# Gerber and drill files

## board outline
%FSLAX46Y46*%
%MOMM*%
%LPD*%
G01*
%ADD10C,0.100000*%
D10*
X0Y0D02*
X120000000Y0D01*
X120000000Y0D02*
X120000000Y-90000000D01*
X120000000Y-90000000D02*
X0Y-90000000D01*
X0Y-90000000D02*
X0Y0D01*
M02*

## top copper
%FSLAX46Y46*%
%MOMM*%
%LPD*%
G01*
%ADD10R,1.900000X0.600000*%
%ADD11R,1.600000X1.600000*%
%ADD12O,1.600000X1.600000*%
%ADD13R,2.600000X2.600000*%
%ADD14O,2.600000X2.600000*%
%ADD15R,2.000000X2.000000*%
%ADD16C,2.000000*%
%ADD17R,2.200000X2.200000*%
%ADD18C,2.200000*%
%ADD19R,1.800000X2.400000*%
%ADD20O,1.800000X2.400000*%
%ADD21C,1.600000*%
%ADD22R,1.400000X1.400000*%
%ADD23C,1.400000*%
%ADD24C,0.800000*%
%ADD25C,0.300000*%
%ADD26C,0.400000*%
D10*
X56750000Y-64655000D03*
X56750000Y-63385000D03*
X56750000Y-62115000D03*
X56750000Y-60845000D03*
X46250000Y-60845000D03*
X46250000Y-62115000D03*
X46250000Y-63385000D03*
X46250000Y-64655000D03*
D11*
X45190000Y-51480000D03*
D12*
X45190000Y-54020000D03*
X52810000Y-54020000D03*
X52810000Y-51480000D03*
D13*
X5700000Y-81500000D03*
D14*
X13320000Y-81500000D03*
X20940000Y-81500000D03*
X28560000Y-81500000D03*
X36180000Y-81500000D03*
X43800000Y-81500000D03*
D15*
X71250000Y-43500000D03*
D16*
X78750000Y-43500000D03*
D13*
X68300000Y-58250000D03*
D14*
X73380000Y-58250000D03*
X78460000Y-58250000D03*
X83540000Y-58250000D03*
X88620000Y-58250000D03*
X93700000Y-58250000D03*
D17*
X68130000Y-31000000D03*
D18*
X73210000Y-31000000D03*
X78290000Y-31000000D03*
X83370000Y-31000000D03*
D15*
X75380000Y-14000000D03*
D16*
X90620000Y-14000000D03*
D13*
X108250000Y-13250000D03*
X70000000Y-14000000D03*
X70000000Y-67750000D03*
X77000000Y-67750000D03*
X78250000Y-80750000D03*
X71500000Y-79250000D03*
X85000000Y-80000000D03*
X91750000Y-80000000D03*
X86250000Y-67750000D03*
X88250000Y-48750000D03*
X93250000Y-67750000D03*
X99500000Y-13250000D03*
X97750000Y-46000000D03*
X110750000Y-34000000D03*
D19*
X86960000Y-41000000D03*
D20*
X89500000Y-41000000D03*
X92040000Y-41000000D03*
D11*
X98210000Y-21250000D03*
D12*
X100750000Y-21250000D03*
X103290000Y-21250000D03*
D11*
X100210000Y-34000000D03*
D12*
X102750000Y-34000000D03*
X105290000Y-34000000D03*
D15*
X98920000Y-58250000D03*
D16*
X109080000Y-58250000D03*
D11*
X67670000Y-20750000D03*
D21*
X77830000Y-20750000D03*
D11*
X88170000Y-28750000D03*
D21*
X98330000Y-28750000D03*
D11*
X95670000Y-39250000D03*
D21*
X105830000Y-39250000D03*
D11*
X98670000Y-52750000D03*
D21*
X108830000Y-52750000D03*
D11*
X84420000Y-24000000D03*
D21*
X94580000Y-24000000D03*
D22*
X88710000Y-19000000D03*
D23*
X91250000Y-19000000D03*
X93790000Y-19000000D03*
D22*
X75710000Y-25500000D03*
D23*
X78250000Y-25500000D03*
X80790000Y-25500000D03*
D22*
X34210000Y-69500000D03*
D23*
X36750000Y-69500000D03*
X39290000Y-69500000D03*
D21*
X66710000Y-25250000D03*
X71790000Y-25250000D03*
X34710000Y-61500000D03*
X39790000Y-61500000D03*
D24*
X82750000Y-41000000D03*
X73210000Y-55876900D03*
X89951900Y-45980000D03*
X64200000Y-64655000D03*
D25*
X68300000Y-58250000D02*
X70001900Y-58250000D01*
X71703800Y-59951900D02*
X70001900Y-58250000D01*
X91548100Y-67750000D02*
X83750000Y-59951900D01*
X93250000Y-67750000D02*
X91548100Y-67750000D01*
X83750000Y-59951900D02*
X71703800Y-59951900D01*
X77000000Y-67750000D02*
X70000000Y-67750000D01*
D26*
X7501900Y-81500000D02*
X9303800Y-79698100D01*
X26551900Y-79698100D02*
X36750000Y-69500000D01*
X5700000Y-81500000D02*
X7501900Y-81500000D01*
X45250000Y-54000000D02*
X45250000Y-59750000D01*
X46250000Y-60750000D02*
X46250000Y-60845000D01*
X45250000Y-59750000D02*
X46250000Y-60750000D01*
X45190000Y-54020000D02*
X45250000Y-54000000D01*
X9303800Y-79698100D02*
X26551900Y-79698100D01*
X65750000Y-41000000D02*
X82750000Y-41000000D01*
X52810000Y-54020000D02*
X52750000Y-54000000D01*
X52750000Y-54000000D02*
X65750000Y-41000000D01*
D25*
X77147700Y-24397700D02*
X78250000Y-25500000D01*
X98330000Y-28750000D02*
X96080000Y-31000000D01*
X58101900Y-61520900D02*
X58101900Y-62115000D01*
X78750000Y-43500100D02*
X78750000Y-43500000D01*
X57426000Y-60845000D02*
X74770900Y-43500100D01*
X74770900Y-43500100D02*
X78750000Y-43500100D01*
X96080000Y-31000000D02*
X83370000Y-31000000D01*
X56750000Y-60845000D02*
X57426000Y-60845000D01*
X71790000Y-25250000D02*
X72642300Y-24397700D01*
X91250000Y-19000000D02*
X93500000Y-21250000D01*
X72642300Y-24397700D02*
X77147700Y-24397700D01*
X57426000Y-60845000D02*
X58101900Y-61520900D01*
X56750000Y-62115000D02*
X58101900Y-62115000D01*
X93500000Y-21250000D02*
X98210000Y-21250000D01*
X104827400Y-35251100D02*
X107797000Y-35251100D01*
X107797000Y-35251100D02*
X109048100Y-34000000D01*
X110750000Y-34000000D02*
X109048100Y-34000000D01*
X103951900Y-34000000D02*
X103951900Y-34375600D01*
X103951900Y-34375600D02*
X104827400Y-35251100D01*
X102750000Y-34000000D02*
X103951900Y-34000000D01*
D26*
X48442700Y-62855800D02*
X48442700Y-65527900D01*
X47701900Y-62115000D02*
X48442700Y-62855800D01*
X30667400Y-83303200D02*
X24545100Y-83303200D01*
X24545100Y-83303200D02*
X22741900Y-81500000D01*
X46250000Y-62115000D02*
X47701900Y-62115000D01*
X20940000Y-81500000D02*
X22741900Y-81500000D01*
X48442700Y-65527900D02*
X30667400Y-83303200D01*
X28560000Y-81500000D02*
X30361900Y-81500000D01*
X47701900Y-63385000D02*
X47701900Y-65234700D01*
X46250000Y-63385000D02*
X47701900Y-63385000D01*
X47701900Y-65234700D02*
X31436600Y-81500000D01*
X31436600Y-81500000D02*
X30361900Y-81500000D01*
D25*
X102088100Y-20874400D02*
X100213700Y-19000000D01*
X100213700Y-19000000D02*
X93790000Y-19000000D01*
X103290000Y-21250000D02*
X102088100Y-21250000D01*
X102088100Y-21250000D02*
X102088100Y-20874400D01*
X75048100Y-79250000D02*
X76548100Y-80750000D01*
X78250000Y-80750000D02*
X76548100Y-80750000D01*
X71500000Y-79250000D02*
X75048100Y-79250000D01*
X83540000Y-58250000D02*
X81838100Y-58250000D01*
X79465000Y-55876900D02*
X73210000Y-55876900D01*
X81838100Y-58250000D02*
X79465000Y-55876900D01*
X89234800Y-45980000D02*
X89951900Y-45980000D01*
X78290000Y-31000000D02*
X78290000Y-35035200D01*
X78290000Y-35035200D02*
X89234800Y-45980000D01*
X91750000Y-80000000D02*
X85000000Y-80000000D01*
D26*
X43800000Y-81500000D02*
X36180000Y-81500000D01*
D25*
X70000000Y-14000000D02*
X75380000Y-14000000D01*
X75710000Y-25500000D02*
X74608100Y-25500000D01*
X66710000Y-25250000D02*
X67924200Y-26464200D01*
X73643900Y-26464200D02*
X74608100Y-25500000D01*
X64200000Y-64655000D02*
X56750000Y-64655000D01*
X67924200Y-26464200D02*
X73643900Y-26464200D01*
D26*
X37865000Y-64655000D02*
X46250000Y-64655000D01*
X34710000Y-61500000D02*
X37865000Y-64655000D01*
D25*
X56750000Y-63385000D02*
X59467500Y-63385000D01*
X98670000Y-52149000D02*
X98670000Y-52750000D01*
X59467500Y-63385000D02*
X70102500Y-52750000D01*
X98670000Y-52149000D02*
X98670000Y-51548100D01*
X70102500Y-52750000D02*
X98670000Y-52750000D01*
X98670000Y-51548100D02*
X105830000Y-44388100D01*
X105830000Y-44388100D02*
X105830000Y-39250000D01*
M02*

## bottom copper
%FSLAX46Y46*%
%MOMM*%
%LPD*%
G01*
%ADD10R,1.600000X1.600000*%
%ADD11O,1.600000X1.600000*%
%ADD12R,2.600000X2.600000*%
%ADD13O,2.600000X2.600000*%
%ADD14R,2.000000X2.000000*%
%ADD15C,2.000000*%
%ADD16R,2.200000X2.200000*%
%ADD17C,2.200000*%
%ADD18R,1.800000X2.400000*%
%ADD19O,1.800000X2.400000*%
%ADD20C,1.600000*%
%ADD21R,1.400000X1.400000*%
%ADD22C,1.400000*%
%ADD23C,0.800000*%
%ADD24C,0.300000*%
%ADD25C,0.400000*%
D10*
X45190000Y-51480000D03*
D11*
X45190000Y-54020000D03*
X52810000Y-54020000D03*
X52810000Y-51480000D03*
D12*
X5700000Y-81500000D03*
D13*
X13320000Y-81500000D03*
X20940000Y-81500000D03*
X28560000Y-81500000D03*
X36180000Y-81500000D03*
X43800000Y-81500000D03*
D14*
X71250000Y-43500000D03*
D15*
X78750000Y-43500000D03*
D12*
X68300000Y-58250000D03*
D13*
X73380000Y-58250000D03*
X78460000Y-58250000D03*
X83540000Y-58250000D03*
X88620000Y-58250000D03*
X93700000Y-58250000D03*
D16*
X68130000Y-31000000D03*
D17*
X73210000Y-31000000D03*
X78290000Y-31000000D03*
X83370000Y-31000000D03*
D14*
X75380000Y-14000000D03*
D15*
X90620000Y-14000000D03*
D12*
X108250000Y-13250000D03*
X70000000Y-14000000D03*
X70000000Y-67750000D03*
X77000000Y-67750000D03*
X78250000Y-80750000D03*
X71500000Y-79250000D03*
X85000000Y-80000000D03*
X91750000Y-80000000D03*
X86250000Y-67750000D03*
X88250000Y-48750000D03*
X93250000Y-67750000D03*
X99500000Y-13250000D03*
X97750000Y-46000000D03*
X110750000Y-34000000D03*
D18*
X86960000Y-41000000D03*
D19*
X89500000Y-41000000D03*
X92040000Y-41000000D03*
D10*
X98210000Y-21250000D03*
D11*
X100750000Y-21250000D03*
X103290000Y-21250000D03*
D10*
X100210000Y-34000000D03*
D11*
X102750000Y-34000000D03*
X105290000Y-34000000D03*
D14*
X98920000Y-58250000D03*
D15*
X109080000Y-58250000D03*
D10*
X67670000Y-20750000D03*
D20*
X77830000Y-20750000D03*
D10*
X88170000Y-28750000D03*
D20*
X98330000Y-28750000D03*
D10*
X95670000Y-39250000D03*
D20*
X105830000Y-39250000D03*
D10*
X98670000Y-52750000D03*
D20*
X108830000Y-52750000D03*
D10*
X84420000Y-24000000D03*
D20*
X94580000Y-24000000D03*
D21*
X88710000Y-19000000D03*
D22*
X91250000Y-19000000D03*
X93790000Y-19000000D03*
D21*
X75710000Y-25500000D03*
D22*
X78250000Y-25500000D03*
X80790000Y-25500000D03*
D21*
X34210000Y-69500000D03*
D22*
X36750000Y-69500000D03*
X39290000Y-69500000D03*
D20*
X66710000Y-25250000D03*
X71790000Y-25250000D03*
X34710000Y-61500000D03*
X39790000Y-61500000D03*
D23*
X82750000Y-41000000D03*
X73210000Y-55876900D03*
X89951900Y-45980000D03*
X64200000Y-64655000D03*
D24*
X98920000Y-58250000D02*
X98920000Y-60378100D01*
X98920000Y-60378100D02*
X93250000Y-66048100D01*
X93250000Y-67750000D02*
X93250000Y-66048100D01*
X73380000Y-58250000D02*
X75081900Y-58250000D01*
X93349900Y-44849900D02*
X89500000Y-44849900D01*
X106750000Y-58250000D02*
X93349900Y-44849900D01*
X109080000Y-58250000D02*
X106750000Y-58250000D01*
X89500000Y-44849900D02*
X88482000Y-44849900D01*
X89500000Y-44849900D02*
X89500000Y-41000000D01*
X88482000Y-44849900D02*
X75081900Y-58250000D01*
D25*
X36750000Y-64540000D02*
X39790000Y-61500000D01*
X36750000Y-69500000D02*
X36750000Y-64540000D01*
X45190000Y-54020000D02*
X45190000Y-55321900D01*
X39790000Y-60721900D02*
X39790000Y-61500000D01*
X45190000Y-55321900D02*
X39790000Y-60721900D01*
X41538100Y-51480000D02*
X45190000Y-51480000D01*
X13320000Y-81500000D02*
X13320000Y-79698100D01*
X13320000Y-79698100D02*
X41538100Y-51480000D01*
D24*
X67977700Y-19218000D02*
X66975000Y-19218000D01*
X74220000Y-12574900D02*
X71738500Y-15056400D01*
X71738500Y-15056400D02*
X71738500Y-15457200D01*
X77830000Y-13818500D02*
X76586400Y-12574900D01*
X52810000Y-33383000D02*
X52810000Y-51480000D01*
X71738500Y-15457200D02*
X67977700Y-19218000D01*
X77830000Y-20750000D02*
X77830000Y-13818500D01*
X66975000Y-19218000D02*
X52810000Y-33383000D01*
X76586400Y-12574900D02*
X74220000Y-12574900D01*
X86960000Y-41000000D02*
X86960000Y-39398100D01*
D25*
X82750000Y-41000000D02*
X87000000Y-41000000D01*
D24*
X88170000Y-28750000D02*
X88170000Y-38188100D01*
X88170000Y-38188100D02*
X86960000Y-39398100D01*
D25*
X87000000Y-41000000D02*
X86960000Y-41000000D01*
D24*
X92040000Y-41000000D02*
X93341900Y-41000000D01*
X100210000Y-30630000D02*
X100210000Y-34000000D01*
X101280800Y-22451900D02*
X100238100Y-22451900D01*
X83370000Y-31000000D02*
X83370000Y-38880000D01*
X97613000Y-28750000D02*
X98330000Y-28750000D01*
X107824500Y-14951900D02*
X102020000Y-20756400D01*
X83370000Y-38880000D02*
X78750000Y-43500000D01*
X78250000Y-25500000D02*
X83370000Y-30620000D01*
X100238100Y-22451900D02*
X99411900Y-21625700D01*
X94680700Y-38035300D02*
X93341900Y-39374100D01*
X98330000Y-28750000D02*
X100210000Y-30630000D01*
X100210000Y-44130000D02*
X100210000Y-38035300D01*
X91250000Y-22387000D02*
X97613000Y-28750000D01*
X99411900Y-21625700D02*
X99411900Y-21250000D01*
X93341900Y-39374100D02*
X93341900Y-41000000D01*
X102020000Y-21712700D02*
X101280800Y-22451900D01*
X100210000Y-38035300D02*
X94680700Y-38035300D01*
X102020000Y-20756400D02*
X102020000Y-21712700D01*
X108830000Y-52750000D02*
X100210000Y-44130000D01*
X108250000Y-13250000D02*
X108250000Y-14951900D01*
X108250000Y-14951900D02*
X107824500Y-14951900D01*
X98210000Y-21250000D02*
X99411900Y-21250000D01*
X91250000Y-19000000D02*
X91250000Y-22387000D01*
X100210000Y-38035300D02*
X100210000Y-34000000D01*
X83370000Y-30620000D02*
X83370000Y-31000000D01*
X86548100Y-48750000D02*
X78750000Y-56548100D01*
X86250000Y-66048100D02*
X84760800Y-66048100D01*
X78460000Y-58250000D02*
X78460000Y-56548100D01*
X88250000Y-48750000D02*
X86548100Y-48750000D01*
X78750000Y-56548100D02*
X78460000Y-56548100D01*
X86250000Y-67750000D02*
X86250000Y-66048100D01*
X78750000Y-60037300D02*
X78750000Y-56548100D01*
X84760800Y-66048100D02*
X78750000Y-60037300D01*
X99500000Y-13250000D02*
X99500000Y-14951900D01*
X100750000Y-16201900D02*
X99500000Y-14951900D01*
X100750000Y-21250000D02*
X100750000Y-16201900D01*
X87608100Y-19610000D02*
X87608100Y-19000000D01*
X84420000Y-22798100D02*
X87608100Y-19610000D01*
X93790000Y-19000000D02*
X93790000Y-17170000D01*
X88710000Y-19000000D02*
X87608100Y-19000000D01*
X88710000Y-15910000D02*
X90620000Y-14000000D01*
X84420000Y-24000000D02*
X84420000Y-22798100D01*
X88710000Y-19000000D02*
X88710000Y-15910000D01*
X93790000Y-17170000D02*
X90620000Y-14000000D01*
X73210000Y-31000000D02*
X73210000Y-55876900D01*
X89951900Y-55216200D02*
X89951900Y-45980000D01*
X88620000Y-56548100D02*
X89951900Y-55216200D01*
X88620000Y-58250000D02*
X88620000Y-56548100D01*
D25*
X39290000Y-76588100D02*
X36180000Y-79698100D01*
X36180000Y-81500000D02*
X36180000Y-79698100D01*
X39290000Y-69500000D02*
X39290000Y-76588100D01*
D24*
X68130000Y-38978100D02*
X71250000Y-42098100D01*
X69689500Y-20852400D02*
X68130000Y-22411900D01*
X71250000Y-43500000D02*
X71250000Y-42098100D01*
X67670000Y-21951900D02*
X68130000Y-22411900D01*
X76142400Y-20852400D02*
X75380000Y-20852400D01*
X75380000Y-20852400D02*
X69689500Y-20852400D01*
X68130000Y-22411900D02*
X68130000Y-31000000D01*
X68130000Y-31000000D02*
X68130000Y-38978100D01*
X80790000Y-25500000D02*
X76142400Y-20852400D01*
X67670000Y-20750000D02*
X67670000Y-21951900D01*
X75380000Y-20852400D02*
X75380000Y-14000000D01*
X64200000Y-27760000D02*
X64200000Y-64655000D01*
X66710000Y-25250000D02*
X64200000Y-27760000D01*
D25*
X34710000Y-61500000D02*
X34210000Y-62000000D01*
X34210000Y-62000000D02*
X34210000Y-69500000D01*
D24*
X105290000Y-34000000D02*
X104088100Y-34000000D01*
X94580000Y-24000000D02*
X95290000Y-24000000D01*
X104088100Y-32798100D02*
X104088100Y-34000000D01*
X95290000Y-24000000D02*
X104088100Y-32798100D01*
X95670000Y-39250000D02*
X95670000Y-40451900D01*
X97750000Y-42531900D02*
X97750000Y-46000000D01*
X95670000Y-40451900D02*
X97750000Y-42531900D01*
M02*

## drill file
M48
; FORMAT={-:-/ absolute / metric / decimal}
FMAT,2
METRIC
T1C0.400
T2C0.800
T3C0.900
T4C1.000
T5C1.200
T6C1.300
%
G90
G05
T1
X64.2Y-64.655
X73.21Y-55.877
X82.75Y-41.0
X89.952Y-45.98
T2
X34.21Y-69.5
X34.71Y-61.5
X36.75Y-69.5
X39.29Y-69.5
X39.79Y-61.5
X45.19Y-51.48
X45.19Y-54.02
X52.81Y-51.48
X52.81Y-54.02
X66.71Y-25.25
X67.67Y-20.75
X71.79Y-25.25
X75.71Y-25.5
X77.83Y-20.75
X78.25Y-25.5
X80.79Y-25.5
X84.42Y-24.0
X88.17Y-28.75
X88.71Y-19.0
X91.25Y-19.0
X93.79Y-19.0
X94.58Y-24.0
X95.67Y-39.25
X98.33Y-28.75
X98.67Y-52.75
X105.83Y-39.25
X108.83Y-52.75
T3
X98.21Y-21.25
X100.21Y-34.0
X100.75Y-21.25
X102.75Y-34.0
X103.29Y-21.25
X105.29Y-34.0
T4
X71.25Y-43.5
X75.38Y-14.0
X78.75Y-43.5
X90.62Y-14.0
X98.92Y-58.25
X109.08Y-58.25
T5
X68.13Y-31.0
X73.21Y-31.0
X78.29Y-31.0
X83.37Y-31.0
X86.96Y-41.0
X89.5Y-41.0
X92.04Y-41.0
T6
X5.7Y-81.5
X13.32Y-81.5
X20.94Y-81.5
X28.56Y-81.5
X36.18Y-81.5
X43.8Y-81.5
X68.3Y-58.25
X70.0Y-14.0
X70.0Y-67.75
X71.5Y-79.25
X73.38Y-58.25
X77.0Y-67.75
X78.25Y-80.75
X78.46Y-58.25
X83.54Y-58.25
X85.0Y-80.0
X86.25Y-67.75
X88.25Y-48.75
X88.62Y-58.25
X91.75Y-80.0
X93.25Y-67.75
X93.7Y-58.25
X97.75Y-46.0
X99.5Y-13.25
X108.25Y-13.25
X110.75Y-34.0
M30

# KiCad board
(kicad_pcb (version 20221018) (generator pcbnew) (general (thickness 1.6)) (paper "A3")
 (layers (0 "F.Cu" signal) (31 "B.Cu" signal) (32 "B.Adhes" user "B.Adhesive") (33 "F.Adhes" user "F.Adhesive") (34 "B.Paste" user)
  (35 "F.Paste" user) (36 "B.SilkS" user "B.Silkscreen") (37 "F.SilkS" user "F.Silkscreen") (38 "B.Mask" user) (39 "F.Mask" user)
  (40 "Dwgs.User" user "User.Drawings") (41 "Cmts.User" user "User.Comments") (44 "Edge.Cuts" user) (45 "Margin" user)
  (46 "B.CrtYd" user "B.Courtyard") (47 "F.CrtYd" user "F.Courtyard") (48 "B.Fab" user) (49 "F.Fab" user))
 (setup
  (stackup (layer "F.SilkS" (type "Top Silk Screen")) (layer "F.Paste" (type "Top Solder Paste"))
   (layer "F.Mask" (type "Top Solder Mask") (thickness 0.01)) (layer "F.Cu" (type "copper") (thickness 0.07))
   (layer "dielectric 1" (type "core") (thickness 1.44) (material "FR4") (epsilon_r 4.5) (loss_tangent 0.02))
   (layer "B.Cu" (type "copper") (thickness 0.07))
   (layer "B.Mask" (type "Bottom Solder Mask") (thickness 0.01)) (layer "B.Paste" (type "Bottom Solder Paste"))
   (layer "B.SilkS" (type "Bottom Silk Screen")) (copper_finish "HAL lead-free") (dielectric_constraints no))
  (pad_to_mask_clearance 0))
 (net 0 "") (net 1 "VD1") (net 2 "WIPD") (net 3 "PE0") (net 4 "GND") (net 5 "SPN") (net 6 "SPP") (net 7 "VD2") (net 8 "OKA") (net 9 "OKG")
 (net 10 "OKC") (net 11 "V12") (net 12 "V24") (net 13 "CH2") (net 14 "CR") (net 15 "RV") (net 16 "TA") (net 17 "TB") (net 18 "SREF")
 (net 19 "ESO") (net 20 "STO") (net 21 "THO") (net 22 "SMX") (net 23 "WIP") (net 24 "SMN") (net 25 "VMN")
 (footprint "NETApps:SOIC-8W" (layer "F.Cu") (at 51.5 62.75 180)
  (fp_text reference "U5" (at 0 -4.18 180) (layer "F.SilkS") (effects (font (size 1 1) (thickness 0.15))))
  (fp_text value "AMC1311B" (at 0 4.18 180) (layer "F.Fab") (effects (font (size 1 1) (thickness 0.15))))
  (pad "1" smd rect (at -5.25 -1.905) (size 1.9 0.6) (layers "F.Cu" "F.Paste" "F.Mask") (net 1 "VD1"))
  (pad "2" smd rect (at -5.25 -0.635) (size 1.9 0.6) (layers "F.Cu" "F.Paste" "F.Mask") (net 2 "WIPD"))
  (pad "3" smd rect (at -5.25 0.635) (size 1.9 0.6) (layers "F.Cu" "F.Paste" "F.Mask") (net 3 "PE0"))
  (pad "4" smd rect (at -5.25 1.905) (size 1.9 0.6) (layers "F.Cu" "F.Paste" "F.Mask") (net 3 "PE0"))
  (pad "5" smd rect (at 5.25 1.905) (size 1.9 0.6) (layers "F.Cu" "F.Paste" "F.Mask") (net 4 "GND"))
  (pad "6" smd rect (at 5.25 0.635) (size 1.9 0.6) (layers "F.Cu" "F.Paste" "F.Mask") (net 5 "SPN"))
  (pad "7" smd rect (at 5.25 -0.635) (size 1.9 0.6) (layers "F.Cu" "F.Paste" "F.Mask") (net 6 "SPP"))
  (pad "8" smd rect (at 5.25 -1.905) (size 1.9 0.6) (layers "F.Cu" "F.Paste" "F.Mask") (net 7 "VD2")))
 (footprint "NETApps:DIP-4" (layer "F.Cu") (at 49 52.75)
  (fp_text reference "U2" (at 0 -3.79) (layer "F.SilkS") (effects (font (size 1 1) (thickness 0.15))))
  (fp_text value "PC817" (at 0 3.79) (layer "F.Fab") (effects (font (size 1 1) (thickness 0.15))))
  (pad "1" thru_hole rect (at -3.81 -1.27) (size 1.6 1.6) (drill 0.8) (layers "*.Cu" "*.Mask") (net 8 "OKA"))
  (pad "2" thru_hole oval (at -3.81 1.27) (size 1.6 1.6) (drill 0.8) (layers "*.Cu" "*.Mask") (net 4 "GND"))
  (pad "3" thru_hole oval (at 3.81 1.27) (size 1.6 1.6) (drill 0.8) (layers "*.Cu" "*.Mask") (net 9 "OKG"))
  (pad "4" thru_hole oval (at 3.81 -1.27) (size 1.6 1.6) (drill 0.8) (layers "*.Cu" "*.Mask") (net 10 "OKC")))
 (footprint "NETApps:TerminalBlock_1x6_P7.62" (layer "F.Cu") (at 24.75 81.5)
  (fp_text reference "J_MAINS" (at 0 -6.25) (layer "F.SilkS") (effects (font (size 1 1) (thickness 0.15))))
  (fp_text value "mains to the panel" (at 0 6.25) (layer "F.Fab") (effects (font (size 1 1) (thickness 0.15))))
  (pad "1" thru_hole rect (at -19.05 0) (size 2.6 2.6) (drill 1.3) (layers "*.Cu" "*.Mask") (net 4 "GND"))
  (pad "2" thru_hole oval (at -11.43 0) (size 2.6 2.6) (drill 1.3) (layers "*.Cu" "*.Mask") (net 8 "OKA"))
  (pad "3" thru_hole oval (at -3.81 0) (size 2.6 2.6) (drill 1.3) (layers "*.Cu" "*.Mask") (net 5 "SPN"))
  (pad "4" thru_hole oval (at 3.81 0) (size 2.6 2.6) (drill 1.3) (layers "*.Cu" "*.Mask") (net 6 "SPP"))
  (pad "5" thru_hole oval (at 11.43 0) (size 2.6 2.6) (drill 1.3) (layers "*.Cu" "*.Mask") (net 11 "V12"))
  (pad "6" thru_hole oval (at 19.05 0) (size 2.6 2.6) (drill 1.3) (layers "*.Cu" "*.Mask") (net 11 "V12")))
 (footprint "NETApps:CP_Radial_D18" (layer "F.Cu") (at 75 43.5)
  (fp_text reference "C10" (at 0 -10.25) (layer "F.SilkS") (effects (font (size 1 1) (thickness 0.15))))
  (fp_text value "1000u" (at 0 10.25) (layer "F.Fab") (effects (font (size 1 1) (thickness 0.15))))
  (pad "1" thru_hole rect (at -3.75 0) (size 2 2) (drill 1) (layers "*.Cu" "*.Mask") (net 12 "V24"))
  (pad "2" thru_hole circle (at 3.75 0) (size 2 2) (drill 1) (layers "*.Cu" "*.Mask") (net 3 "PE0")))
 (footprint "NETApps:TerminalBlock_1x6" (layer "F.Cu") (at 81 58.25)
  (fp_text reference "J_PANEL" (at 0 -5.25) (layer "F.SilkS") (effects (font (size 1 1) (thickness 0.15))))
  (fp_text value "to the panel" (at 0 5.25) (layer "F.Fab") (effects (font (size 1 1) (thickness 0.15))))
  (pad "1" thru_hole rect (at -12.7 0) (size 2.6 2.6) (drill 1.3) (layers "*.Cu" "*.Mask") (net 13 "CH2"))
  (pad "2" thru_hole oval (at -7.62 0) (size 2.6 2.6) (drill 1.3) (layers "*.Cu" "*.Mask") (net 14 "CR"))
  (pad "3" thru_hole oval (at -2.54 0) (size 2.6 2.6) (drill 1.3) (layers "*.Cu" "*.Mask") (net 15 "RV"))
  (pad "4" thru_hole oval (at 2.54 0) (size 2.6 2.6) (drill 1.3) (layers "*.Cu" "*.Mask") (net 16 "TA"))
  (pad "5" thru_hole oval (at 7.62 0) (size 2.6 2.6) (drill 1.3) (layers "*.Cu" "*.Mask") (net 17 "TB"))
  (pad "6" thru_hole oval (at 12.7 0) (size 2.6 2.6) (drill 1.3) (layers "*.Cu" "*.Mask")))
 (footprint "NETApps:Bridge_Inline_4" (layer "F.Cu") (at 75.75 31)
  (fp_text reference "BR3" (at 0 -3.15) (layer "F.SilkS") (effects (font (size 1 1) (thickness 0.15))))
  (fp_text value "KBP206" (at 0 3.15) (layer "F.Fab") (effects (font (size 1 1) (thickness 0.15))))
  (pad "1" thru_hole rect (at -7.62 0) (size 2.2 2.2) (drill 1.2) (layers "*.Cu" "*.Mask") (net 12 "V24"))
  (pad "2" thru_hole circle (at -2.54 0) (size 2.2 2.2) (drill 1.2) (layers "*.Cu" "*.Mask") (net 16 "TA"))
  (pad "3" thru_hole circle (at 2.54 0) (size 2.2 2.2) (drill 1.2) (layers "*.Cu" "*.Mask") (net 17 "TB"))
  (pad "4" thru_hole circle (at 7.62 0) (size 2.2 2.2) (drill 1.2) (layers "*.Cu" "*.Mask") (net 3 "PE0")))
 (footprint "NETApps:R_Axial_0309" (layer "F.Cu") (at 83 14)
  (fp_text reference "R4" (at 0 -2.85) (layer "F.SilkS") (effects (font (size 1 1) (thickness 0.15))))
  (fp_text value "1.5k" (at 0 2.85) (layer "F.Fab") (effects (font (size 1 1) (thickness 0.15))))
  (pad "1" thru_hole rect (at -7.62 0) (size 2 2) (drill 1) (layers "*.Cu" "*.Mask") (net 12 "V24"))
  (pad "2" thru_hole circle (at 7.62 0) (size 2 2) (drill 1) (layers "*.Cu" "*.Mask") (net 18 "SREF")))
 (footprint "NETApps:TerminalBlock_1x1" (layer "F.Cu") (at 108.25 13.25)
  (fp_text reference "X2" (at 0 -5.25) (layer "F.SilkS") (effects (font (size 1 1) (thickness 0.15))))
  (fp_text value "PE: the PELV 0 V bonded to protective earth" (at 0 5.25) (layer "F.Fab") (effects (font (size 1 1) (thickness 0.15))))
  (pad "1" thru_hole rect (at 0 0) (size 2.6 2.6) (drill 1.3) (layers "*.Cu" "*.Mask") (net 3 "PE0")))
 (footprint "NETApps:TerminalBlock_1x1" (layer "F.Cu") (at 70 14)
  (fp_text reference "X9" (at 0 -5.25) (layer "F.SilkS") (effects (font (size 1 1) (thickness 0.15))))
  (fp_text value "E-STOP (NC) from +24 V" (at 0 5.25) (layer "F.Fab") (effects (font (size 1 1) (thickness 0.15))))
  (pad "1" thru_hole rect (at 0 0) (size 2.6 2.6) (drill 1.3) (layers "*.Cu" "*.Mask") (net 12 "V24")))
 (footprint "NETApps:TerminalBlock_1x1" (layer "F.Cu") (at 70 67.75)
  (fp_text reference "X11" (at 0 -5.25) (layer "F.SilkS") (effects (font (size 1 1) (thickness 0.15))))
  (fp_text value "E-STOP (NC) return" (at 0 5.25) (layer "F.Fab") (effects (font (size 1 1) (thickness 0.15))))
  (pad "1" thru_hole rect (at 0 0) (size 2.6 2.6) (drill 1.3) (layers "*.Cu" "*.Mask") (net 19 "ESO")))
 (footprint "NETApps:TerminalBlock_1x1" (layer "F.Cu") (at 77 67.75)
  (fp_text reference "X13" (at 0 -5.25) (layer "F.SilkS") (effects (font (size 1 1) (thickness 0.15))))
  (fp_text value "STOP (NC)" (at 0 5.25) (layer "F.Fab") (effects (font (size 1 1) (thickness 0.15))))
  (pad "1" thru_hole rect (at 0 0) (size 2.6 2.6) (drill 1.3) (layers "*.Cu" "*.Mask") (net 19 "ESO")))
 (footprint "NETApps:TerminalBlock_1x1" (layer "F.Cu") (at 78.25 80.75)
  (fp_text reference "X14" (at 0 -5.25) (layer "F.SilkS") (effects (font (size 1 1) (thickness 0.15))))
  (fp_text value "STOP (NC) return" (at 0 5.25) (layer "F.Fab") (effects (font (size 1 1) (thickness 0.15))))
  (pad "1" thru_hole rect (at 0 0) (size 2.6 2.6) (drill 1.3) (layers "*.Cu" "*.Mask") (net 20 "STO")))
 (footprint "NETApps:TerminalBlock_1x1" (layer "F.Cu") (at 71.5 79.25)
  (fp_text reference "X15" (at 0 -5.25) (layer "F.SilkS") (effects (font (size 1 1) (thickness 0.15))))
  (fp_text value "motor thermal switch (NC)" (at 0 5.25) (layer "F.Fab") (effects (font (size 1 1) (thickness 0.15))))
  (pad "1" thru_hole rect (at 0 0) (size 2.6 2.6) (drill 1.3) (layers "*.Cu" "*.Mask") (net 20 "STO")))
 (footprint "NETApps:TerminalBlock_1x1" (layer "F.Cu") (at 85 80)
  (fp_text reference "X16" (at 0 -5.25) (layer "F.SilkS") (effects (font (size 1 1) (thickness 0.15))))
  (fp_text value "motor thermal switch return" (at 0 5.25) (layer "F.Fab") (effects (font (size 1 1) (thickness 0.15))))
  (pad "1" thru_hole rect (at 0 0) (size 2.6 2.6) (drill 1.3) (layers "*.Cu" "*.Mask") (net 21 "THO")))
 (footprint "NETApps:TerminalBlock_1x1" (layer "F.Cu") (at 91.75 80)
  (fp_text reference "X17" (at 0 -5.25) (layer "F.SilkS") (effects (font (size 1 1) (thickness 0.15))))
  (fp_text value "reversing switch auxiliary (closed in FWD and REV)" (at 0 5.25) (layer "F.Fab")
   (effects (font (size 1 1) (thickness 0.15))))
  (pad "1" thru_hole rect (at 0 0) (size 2.6 2.6) (drill 1.3) (layers "*.Cu" "*.Mask") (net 21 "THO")))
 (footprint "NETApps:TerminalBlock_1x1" (layer "F.Cu") (at 86.25 67.75)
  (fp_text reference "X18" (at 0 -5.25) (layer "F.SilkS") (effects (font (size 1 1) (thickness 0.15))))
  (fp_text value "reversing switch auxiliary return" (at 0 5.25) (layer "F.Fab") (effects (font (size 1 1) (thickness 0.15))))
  (pad "1" thru_hole rect (at 0 0) (size 2.6 2.6) (drill 1.3) (layers "*.Cu" "*.Mask") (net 15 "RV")))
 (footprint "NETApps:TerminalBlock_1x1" (layer "F.Cu") (at 88.25 48.75)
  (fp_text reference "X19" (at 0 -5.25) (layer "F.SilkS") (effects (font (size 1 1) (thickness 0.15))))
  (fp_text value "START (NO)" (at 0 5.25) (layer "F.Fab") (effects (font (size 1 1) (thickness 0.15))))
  (pad "1" thru_hole rect (at 0 0) (size 2.6 2.6) (drill 1.3) (layers "*.Cu" "*.Mask") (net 15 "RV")))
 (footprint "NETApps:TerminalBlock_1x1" (layer "F.Cu") (at 93.25 67.75)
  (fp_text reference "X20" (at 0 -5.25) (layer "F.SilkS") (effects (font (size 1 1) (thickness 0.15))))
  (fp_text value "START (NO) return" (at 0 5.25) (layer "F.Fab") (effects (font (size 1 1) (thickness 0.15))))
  (pad "1" thru_hole rect (at 0 0) (size 2.6 2.6) (drill 1.3) (layers "*.Cu" "*.Mask") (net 13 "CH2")))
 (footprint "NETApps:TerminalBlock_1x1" (layer "F.Cu") (at 99.5 13.25)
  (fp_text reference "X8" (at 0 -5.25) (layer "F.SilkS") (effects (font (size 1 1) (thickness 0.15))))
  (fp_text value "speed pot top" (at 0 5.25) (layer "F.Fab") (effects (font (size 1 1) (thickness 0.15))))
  (pad "1" thru_hole rect (at 0 0) (size 2.6 2.6) (drill 1.3) (layers "*.Cu" "*.Mask") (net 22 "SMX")))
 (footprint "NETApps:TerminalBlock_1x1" (layer "F.Cu") (at 97.75 46)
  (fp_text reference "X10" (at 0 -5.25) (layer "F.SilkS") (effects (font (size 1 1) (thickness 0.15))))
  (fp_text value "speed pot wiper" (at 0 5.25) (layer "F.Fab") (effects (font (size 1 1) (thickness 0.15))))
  (pad "1" thru_hole rect (at 0 0) (size 2.6 2.6) (drill 1.3) (layers "*.Cu" "*.Mask") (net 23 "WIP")))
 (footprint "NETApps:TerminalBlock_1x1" (layer "F.Cu") (at 110.75 34)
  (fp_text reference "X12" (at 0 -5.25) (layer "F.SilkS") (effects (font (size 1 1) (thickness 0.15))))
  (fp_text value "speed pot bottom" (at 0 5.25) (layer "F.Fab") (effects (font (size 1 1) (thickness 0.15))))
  (pad "1" thru_hole rect (at 0 0) (size 2.6 2.6) (drill 1.3) (layers "*.Cu" "*.Mask") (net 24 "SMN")))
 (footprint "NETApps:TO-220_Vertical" (layer "F.Cu") (at 89.5 41)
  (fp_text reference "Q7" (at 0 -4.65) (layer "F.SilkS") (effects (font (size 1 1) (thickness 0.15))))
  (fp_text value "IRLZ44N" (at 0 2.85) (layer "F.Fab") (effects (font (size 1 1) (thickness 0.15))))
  (pad "1" thru_hole rect (at -2.54 0) (size 1.8 2.4) (drill 1.2) (layers "*.Cu" "*.Mask") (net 9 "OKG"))
  (pad "2" thru_hole oval (at 0 0) (size 1.8 2.4) (drill 1.2) (layers "*.Cu" "*.Mask") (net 14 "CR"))
  (pad "3" thru_hole oval (at 2.54 0) (size 1.8 2.4) (drill 1.2) (layers "*.Cu" "*.Mask") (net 3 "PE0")))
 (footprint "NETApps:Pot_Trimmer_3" (layer "F.Cu") (at 100.75 21.25)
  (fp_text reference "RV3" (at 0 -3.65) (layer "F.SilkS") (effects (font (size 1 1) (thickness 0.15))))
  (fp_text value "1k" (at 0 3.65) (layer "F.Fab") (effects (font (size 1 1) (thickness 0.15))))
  (pad "1" thru_hole rect (at -2.54 0) (size 1.6 1.6) (drill 0.9) (layers "*.Cu" "*.Mask") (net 3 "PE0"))
  (pad "2" thru_hole oval (at 0 0) (size 1.6 1.6) (drill 0.9) (layers "*.Cu" "*.Mask") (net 22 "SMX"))
  (pad "3" thru_hole oval (at 2.54 0) (size 1.6 1.6) (drill 0.9) (layers "*.Cu" "*.Mask") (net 18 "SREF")))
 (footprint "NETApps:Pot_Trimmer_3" (layer "F.Cu") (at 102.75 34)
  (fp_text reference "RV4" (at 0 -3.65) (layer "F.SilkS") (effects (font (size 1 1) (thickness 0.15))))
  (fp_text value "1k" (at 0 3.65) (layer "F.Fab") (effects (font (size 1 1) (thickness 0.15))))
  (pad "1" thru_hole rect (at -2.54 0) (size 1.6 1.6) (drill 0.9) (layers "*.Cu" "*.Mask") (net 3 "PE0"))
  (pad "2" thru_hole oval (at 0 0) (size 1.6 1.6) (drill 0.9) (layers "*.Cu" "*.Mask") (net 24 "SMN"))
  (pad "3" thru_hole oval (at 2.54 0) (size 1.6 1.6) (drill 0.9) (layers "*.Cu" "*.Mask") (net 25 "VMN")))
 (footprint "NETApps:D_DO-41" (layer "F.Cu") (at 104 58.25)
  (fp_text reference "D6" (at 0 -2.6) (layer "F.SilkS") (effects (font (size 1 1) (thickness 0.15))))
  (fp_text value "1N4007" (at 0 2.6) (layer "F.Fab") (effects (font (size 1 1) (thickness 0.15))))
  (pad "1" thru_hole rect (at -5.08 0) (size 2 2) (drill 1) (layers "*.Cu" "*.Mask") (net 13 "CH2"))
  (pad "2" thru_hole circle (at 5.08 0) (size 2 2) (drill 1) (layers "*.Cu" "*.Mask") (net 14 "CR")))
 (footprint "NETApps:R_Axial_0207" (layer "F.Cu") (at 72.75 20.75)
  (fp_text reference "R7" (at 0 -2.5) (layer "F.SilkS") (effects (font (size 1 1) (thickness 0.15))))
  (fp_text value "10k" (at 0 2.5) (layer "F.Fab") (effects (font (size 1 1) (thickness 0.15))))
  (pad "1" thru_hole rect (at -5.08 0) (size 1.6 1.6) (drill 0.8) (layers "*.Cu" "*.Mask") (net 12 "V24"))
  (pad "2" thru_hole circle (at 5.08 0) (size 1.6 1.6) (drill 0.8) (layers "*.Cu" "*.Mask") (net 10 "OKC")))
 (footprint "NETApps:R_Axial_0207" (layer "F.Cu") (at 93.25 28.75)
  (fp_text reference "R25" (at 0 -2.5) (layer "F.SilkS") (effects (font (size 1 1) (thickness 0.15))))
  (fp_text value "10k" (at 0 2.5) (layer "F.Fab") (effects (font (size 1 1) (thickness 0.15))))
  (pad "1" thru_hole rect (at -5.08 0) (size 1.6 1.6) (drill 0.8) (layers "*.Cu" "*.Mask") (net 9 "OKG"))
  (pad "2" thru_hole circle (at 5.08 0) (size 1.6 1.6) (drill 0.8) (layers "*.Cu" "*.Mask") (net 3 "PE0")))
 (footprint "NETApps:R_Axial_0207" (layer "F.Cu") (at 100.75 39.25)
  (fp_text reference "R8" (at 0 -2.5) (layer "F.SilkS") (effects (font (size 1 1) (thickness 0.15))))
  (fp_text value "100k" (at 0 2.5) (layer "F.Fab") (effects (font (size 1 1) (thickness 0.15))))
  (pad "1" thru_hole rect (at -5.08 0) (size 1.6 1.6) (drill 0.8) (layers "*.Cu" "*.Mask") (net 23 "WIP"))
  (pad "2" thru_hole circle (at 5.08 0) (size 1.6 1.6) (drill 0.8) (layers "*.Cu" "*.Mask") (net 2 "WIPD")))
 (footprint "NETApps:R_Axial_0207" (layer "F.Cu") (at 103.75 52.75)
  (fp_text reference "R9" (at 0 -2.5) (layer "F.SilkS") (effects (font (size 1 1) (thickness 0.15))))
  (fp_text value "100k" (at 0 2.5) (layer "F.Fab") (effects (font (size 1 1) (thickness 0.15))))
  (pad "1" thru_hole rect (at -5.08 0) (size 1.6 1.6) (drill 0.8) (layers "*.Cu" "*.Mask") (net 2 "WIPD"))
  (pad "2" thru_hole circle (at 5.08 0) (size 1.6 1.6) (drill 0.8) (layers "*.Cu" "*.Mask") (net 3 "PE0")))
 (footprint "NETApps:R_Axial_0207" (layer "F.Cu") (at 89.5 24)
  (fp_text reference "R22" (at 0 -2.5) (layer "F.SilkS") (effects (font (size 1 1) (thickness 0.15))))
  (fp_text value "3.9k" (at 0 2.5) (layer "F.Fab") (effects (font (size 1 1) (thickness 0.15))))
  (pad "1" thru_hole rect (at -5.08 0) (size 1.6 1.6) (drill 0.8) (layers "*.Cu" "*.Mask") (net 18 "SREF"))
  (pad "2" thru_hole circle (at 5.08 0) (size 1.6 1.6) (drill 0.8) (layers "*.Cu" "*.Mask") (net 25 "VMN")))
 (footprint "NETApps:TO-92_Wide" (layer "F.Cu") (at 91.25 19)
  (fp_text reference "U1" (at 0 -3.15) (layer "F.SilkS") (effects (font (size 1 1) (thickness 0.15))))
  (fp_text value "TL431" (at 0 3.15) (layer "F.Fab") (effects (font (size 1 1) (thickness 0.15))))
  (pad "1" thru_hole rect (at -2.54 0) (size 1.4 1.4) (drill 0.8) (layers "*.Cu" "*.Mask") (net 18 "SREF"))
  (pad "2" thru_hole circle (at 0 0) (size 1.4 1.4) (drill 0.8) (layers "*.Cu" "*.Mask") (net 3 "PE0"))
  (pad "3" thru_hole circle (at 2.54 0) (size 1.4 1.4) (drill 0.8) (layers "*.Cu" "*.Mask") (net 18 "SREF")))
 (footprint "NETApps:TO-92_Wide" (layer "F.Cu") (at 78.25 25.5)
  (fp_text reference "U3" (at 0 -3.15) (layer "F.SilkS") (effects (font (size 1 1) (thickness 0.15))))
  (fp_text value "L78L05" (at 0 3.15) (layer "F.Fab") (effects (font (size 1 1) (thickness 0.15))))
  (pad "1" thru_hole rect (at -2.54 0) (size 1.4 1.4) (drill 0.8) (layers "*.Cu" "*.Mask") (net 1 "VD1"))
  (pad "2" thru_hole circle (at 0 0) (size 1.4 1.4) (drill 0.8) (layers "*.Cu" "*.Mask") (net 3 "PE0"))
  (pad "3" thru_hole circle (at 2.54 0) (size 1.4 1.4) (drill 0.8) (layers "*.Cu" "*.Mask") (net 12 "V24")))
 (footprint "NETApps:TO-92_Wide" (layer "F.Cu") (at 36.75 69.5)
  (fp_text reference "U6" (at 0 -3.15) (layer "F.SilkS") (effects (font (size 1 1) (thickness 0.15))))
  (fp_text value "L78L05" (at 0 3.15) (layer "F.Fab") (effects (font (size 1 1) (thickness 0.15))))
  (pad "1" thru_hole rect (at -2.54 0) (size 1.4 1.4) (drill 0.8) (layers "*.Cu" "*.Mask") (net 7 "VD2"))
  (pad "2" thru_hole circle (at 0 0) (size 1.4 1.4) (drill 0.8) (layers "*.Cu" "*.Mask") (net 4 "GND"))
  (pad "3" thru_hole circle (at 2.54 0) (size 1.4 1.4) (drill 0.8) (layers "*.Cu" "*.Mask") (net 11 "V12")))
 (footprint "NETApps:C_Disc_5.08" (layer "F.Cu") (at 69.25 25.25)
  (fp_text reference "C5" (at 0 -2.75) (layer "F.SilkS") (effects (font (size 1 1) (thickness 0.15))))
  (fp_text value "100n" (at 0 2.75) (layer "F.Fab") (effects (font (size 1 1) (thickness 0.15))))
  (pad "1" thru_hole circle (at -2.54 0) (size 1.6 1.6) (drill 0.8) (layers "*.Cu" "*.Mask") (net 1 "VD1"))
  (pad "2" thru_hole circle (at 2.54 0) (size 1.6 1.6) (drill 0.8) (layers "*.Cu" "*.Mask") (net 3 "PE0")))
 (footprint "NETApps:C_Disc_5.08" (layer "F.Cu") (at 37.25 61.5)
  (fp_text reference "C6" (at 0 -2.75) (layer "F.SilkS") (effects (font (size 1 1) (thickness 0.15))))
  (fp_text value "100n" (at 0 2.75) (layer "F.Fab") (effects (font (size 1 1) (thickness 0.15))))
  (pad "1" thru_hole circle (at -2.54 0) (size 1.6 1.6) (drill 0.8) (layers "*.Cu" "*.Mask") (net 7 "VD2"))
  (pad "2" thru_hole circle (at 2.54 0) (size 1.6 1.6) (drill 0.8) (layers "*.Cu" "*.Mask") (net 4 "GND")))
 (gr_line (start 0 0) (end 120 0) (stroke (width 0.1) (type solid)) (layer "Edge.Cuts"))
 (gr_line (start 120 0) (end 120 90) (stroke (width 0.1) (type solid)) (layer "Edge.Cuts"))
 (gr_line (start 120 90) (end 0 90) (stroke (width 0.1) (type solid)) (layer "Edge.Cuts"))
 (gr_line (start 0 90) (end 0 0) (stroke (width 0.1) (type solid)) (layer "Edge.Cuts"))
 (segment (start 68.3 58.25) (end 70.0019 58.25) (width 0.3) (layer "F.Cu") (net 13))
 (segment (start 71.7038 59.9519) (end 70.0019 58.25) (width 0.3) (layer "F.Cu") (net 13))
 (segment (start 91.5481 67.75) (end 83.75 59.9519) (width 0.3) (layer "F.Cu") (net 13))
 (segment (start 93.25 67.75) (end 91.5481 67.75) (width 0.3) (layer "F.Cu") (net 13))
 (segment (start 83.75 59.9519) (end 71.7038 59.9519) (width 0.3) (layer "F.Cu") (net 13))
 (segment (start 98.92 58.25) (end 98.92 60.3781) (width 0.3) (layer "B.Cu") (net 13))
 (segment (start 98.92 60.3781) (end 93.25 66.0481) (width 0.3) (layer "B.Cu") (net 13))
 (segment (start 93.25 67.75) (end 93.25 66.0481) (width 0.3) (layer "B.Cu") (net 13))
 (segment (start 73.38 58.25) (end 75.0819 58.25) (width 0.3) (layer "B.Cu") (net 14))
 (segment (start 93.3499 44.8499) (end 89.5 44.8499) (width 0.3) (layer "B.Cu") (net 14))
 (segment (start 106.75 58.25) (end 93.3499 44.8499) (width 0.3) (layer "B.Cu") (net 14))
 (segment (start 109.08 58.25) (end 106.75 58.25) (width 0.3) (layer "B.Cu") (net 14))
 (segment (start 89.5 44.8499) (end 88.482 44.8499) (width 0.3) (layer "B.Cu") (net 14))
 (segment (start 89.5 44.8499) (end 89.5 41) (width 0.3) (layer "B.Cu") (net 14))
 (segment (start 88.482 44.8499) (end 75.0819 58.25) (width 0.3) (layer "B.Cu") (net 14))
 (segment (start 77 67.75) (end 70 67.75) (width 0.3) (layer "F.Cu") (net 19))
 (segment locked (start 7.5019 81.5) (end 9.3038 79.6981) (width 0.4) (layer "F.Cu") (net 4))
 (segment locked (start 26.5519 79.6981) (end 36.75 69.5) (width 0.4) (layer "F.Cu") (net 4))
 (segment locked (start 5.7 81.5) (end 7.5019 81.5) (width 0.4) (layer "F.Cu") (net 4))
 (segment locked (start 45.25 54) (end 45.25 59.75) (width 0.4) (layer "F.Cu") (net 4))
 (segment locked (start 46.25 60.75) (end 46.25 60.845) (width 0.4) (layer "F.Cu") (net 4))
 (segment locked (start 45.25 59.75) (end 46.25 60.75) (width 0.4) (layer "F.Cu") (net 4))
 (segment locked (start 45.19 54.02) (end 45.25 54) (width 0.4) (layer "F.Cu") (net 4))
 (segment locked (start 9.3038 79.6981) (end 26.5519 79.6981) (width 0.4) (layer "F.Cu") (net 4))
 (segment locked (start 36.75 64.54) (end 39.79 61.5) (width 0.4) (layer "B.Cu") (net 4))
 (segment locked (start 36.75 69.5) (end 36.75 64.54) (width 0.4) (layer "B.Cu") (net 4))
 (segment locked (start 45.19 54.02) (end 45.19 55.3219) (width 0.4) (layer "B.Cu") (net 4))
 (segment locked (start 39.79 60.7219) (end 39.79 61.5) (width 0.4) (layer "B.Cu") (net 4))
 (segment locked (start 45.19 55.3219) (end 39.79 60.7219) (width 0.4) (layer "B.Cu") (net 4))
 (segment locked (start 41.5381 51.48) (end 45.19 51.48) (width 0.4) (layer "B.Cu") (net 8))
 (segment locked (start 13.32 81.5) (end 13.32 79.6981) (width 0.4) (layer "B.Cu") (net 8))
 (segment locked (start 13.32 79.6981) (end 41.5381 51.48) (width 0.4) (layer "B.Cu") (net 8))
 (segment (start 67.9777 19.218) (end 66.975 19.218) (width 0.3) (layer "B.Cu") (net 10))
 (segment (start 74.22 12.5749) (end 71.7385 15.0564) (width 0.3) (layer "B.Cu") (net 10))
 (segment (start 71.7385 15.0564) (end 71.7385 15.4572) (width 0.3) (layer "B.Cu") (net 10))
 (segment (start 77.83 13.8185) (end 76.5864 12.5749) (width 0.3) (layer "B.Cu") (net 10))
 (segment (start 52.81 33.383) (end 52.81 51.48) (width 0.3) (layer "B.Cu") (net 10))
 (segment (start 71.7385 15.4572) (end 67.9777 19.218) (width 0.3) (layer "B.Cu") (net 10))
 (segment (start 77.83 20.75) (end 77.83 13.8185) (width 0.3) (layer "B.Cu") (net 10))
 (segment (start 66.975 19.218) (end 52.81 33.383) (width 0.3) (layer "B.Cu") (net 10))
 (segment (start 76.5864 12.5749) (end 74.22 12.5749) (width 0.3) (layer "B.Cu") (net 10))
 (segment locked (start 65.75 41) (end 82.75 41) (width 0.4) (layer "F.Cu") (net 9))
 (segment locked (start 52.81 54.02) (end 52.75 54) (width 0.4) (layer "F.Cu") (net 9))
 (segment locked (start 52.75 54) (end 65.75 41) (width 0.4) (layer "F.Cu") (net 9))
 (via locked (at 82.75 41) (size 0.8) (drill 0.4) (layers "F.Cu" "B.Cu") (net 9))
 (segment (start 86.96 41) (end 86.96 39.3981) (width 0.3) (layer "B.Cu") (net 9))
 (segment locked (start 82.75 41) (end 87 41) (width 0.4) (layer "B.Cu") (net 9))
 (segment (start 88.17 28.75) (end 88.17 38.1881) (width 0.3) (layer "B.Cu") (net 9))
 (segment (start 88.17 38.1881) (end 86.96 39.3981) (width 0.3) (layer "B.Cu") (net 9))
 (segment locked (start 87 41) (end 86.96 41) (width 0.4) (layer "B.Cu") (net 9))
 (segment (start 77.1477 24.3977) (end 78.25 25.5) (width 0.3) (layer "F.Cu") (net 3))
 (segment (start 98.33 28.75) (end 96.08 31) (width 0.3) (layer "F.Cu") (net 3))
 (segment (start 58.1019 61.5209) (end 58.1019 62.115) (width 0.3) (layer "F.Cu") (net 3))
 (segment (start 78.75 43.5001) (end 78.75 43.5) (width 0.3) (layer "F.Cu") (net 3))
 (segment (start 57.426 60.845) (end 74.7709 43.5001) (width 0.3) (layer "F.Cu") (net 3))
 (segment (start 74.7709 43.5001) (end 78.75 43.5001) (width 0.3) (layer "F.Cu") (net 3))
 (segment (start 96.08 31) (end 83.37 31) (width 0.3) (layer "F.Cu") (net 3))
 (segment (start 56.75 60.845) (end 57.426 60.845) (width 0.3) (layer "F.Cu") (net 3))
 (segment (start 71.79 25.25) (end 72.6423 24.3977) (width 0.3) (layer "F.Cu") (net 3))
 (segment (start 91.25 19) (end 93.5 21.25) (width 0.3) (layer "F.Cu") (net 3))
 (segment (start 72.6423 24.3977) (end 77.1477 24.3977) (width 0.3) (layer "F.Cu") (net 3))
 (segment (start 57.426 60.845) (end 58.1019 61.5209) (width 0.3) (layer "F.Cu") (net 3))
 (segment (start 56.75 62.115) (end 58.1019 62.115) (width 0.3) (layer "F.Cu") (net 3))
 (segment (start 93.5 21.25) (end 98.21 21.25) (width 0.3) (layer "F.Cu") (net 3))
 (segment (start 92.04 41) (end 93.3419 41) (width 0.3) (layer "B.Cu") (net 3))
 (segment (start 100.21 30.63) (end 100.21 34) (width 0.3) (layer "B.Cu") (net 3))
 (segment (start 101.2808 22.4519) (end 100.2381 22.4519) (width 0.3) (layer "B.Cu") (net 3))
 (segment (start 83.37 31) (end 83.37 38.88) (width 0.3) (layer "B.Cu") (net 3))
 (segment (start 97.613 28.75) (end 98.33 28.75) (width 0.3) (layer "B.Cu") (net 3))
 (segment (start 107.8245 14.9519) (end 102.02 20.7564) (width 0.3) (layer "B.Cu") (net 3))
 (segment (start 83.37 38.88) (end 78.75 43.5) (width 0.3) (layer "B.Cu") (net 3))
 (segment (start 78.25 25.5) (end 83.37 30.62) (width 0.3) (layer "B.Cu") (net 3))
 (segment (start 100.2381 22.4519) (end 99.4119 21.6257) (width 0.3) (layer "B.Cu") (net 3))
 (segment (start 94.6807 38.0353) (end 93.3419 39.3741) (width 0.3) (layer "B.Cu") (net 3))
 (segment (start 98.33 28.75) (end 100.21 30.63) (width 0.3) (layer "B.Cu") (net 3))
 (segment (start 100.21 44.13) (end 100.21 38.0353) (width 0.3) (layer "B.Cu") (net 3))
 (segment (start 91.25 22.387) (end 97.613 28.75) (width 0.3) (layer "B.Cu") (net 3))
 (segment (start 99.4119 21.6257) (end 99.4119 21.25) (width 0.3) (layer "B.Cu") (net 3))
 (segment (start 93.3419 39.3741) (end 93.3419 41) (width 0.3) (layer "B.Cu") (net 3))
 (segment (start 102.02 21.7127) (end 101.2808 22.4519) (width 0.3) (layer "B.Cu") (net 3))
 (segment (start 100.21 38.0353) (end 94.6807 38.0353) (width 0.3) (layer "B.Cu") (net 3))
 (segment (start 102.02 20.7564) (end 102.02 21.7127) (width 0.3) (layer "B.Cu") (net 3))
 (segment (start 108.83 52.75) (end 100.21 44.13) (width 0.3) (layer "B.Cu") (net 3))
 (segment (start 108.25 13.25) (end 108.25 14.9519) (width 0.3) (layer "B.Cu") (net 3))
 (segment (start 108.25 14.9519) (end 107.8245 14.9519) (width 0.3) (layer "B.Cu") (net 3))
 (segment (start 98.21 21.25) (end 99.4119 21.25) (width 0.3) (layer "B.Cu") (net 3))
 (segment (start 91.25 19) (end 91.25 22.387) (width 0.3) (layer "B.Cu") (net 3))
 (segment (start 100.21 38.0353) (end 100.21 34) (width 0.3) (layer "B.Cu") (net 3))
 (segment (start 83.37 30.62) (end 83.37 31) (width 0.3) (layer "B.Cu") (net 3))
 (segment (start 86.5481 48.75) (end 78.75 56.5481) (width 0.3) (layer "B.Cu") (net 15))
 (segment (start 86.25 66.0481) (end 84.7608 66.0481) (width 0.3) (layer "B.Cu") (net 15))
 (segment (start 78.46 58.25) (end 78.46 56.5481) (width 0.3) (layer "B.Cu") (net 15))
 (segment (start 88.25 48.75) (end 86.5481 48.75) (width 0.3) (layer "B.Cu") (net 15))
 (segment (start 78.75 56.5481) (end 78.46 56.5481) (width 0.3) (layer "B.Cu") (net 15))
 (segment (start 86.25 67.75) (end 86.25 66.0481) (width 0.3) (layer "B.Cu") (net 15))
 (segment (start 78.75 60.0373) (end 78.75 56.5481) (width 0.3) (layer "B.Cu") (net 15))
 (segment (start 84.7608 66.0481) (end 78.75 60.0373) (width 0.3) (layer "B.Cu") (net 15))
 (segment (start 104.8274 35.2511) (end 107.797 35.2511) (width 0.3) (layer "F.Cu") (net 24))
 (segment (start 107.797 35.2511) (end 109.0481 34) (width 0.3) (layer "F.Cu") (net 24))
 (segment (start 110.75 34) (end 109.0481 34) (width 0.3) (layer "F.Cu") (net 24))
 (segment (start 103.9519 34) (end 103.9519 34.3756) (width 0.3) (layer "F.Cu") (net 24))
 (segment (start 103.9519 34.3756) (end 104.8274 35.2511) (width 0.3) (layer "F.Cu") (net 24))
 (segment (start 102.75 34) (end 103.9519 34) (width 0.3) (layer "F.Cu") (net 24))
 (segment (start 99.5 13.25) (end 99.5 14.9519) (width 0.3) (layer "B.Cu") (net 22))
 (segment (start 100.75 16.2019) (end 99.5 14.9519) (width 0.3) (layer "B.Cu") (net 22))
 (segment (start 100.75 21.25) (end 100.75 16.2019) (width 0.3) (layer "B.Cu") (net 22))
 (segment locked (start 48.4427 62.8558) (end 48.4427 65.5279) (width 0.4) (layer "F.Cu") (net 5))
 (segment locked (start 47.7019 62.115) (end 48.4427 62.8558) (width 0.4) (layer "F.Cu") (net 5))
 (segment locked (start 30.6674 83.3032) (end 24.5451 83.3032) (width 0.4) (layer "F.Cu") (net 5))
 (segment locked (start 24.5451 83.3032) (end 22.7419 81.5) (width 0.4) (layer "F.Cu") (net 5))
 (segment locked (start 46.25 62.115) (end 47.7019 62.115) (width 0.4) (layer "F.Cu") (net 5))
 (segment locked (start 20.94 81.5) (end 22.7419 81.5) (width 0.4) (layer "F.Cu") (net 5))
 (segment locked (start 48.4427 65.5279) (end 30.6674 83.3032) (width 0.4) (layer "F.Cu") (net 5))
 (segment locked (start 28.56 81.5) (end 30.3619 81.5) (width 0.4) (layer "F.Cu") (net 6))
 (segment locked (start 47.7019 63.385) (end 47.7019 65.2347) (width 0.4) (layer "F.Cu") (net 6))
 (segment locked (start 46.25 63.385) (end 47.7019 63.385) (width 0.4) (layer "F.Cu") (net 6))
 (segment locked (start 47.7019 65.2347) (end 31.4366 81.5) (width 0.4) (layer "F.Cu") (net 6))
 (segment locked (start 31.4366 81.5) (end 30.3619 81.5) (width 0.4) (layer "F.Cu") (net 6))
 (segment (start 102.0881 20.8744) (end 100.2137 19) (width 0.3) (layer "F.Cu") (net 18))
 (segment (start 100.2137 19) (end 93.79 19) (width 0.3) (layer "F.Cu") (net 18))
 (segment (start 103.29 21.25) (end 102.0881 21.25) (width 0.3) (layer "F.Cu") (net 18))
 (segment (start 102.0881 21.25) (end 102.0881 20.8744) (width 0.3) (layer "F.Cu") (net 18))
 (segment (start 87.6081 19.61) (end 87.6081 19) (width 0.3) (layer "B.Cu") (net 18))
 (segment (start 84.42 22.7981) (end 87.6081 19.61) (width 0.3) (layer "B.Cu") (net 18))
 (segment (start 93.79 19) (end 93.79 17.17) (width 0.3) (layer "B.Cu") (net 18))
 (segment (start 88.71 19) (end 87.6081 19) (width 0.3) (layer "B.Cu") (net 18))
 (segment (start 88.71 15.91) (end 90.62 14) (width 0.3) (layer "B.Cu") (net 18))
 (segment (start 84.42 24) (end 84.42 22.7981) (width 0.3) (layer "B.Cu") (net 18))
 (segment (start 88.71 19) (end 88.71 15.91) (width 0.3) (layer "B.Cu") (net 18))
 (segment (start 93.79 17.17) (end 90.62 14) (width 0.3) (layer "B.Cu") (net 18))
 (segment (start 75.0481 79.25) (end 76.5481 80.75) (width 0.3) (layer "F.Cu") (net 20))
 (segment (start 78.25 80.75) (end 76.5481 80.75) (width 0.3) (layer "F.Cu") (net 20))
 (segment (start 71.5 79.25) (end 75.0481 79.25) (width 0.3) (layer "F.Cu") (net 20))
 (segment (start 83.54 58.25) (end 81.8381 58.25) (width 0.3) (layer "F.Cu") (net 16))
 (segment (start 79.465 55.8769) (end 73.21 55.8769) (width 0.3) (layer "F.Cu") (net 16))
 (segment (start 81.8381 58.25) (end 79.465 55.8769) (width 0.3) (layer "F.Cu") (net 16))
 (via (at 73.21 55.8769) (size 0.8) (drill 0.4) (layers "F.Cu" "B.Cu") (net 16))
 (segment (start 73.21 31) (end 73.21 55.8769) (width 0.3) (layer "B.Cu") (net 16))
 (segment (start 89.2348 45.98) (end 89.9519 45.98) (width 0.3) (layer "F.Cu") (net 17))
 (segment (start 78.29 31) (end 78.29 35.0352) (width 0.3) (layer "F.Cu") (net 17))
 (segment (start 78.29 35.0352) (end 89.2348 45.98) (width 0.3) (layer "F.Cu") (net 17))
 (via (at 89.9519 45.98) (size 0.8) (drill 0.4) (layers "F.Cu" "B.Cu") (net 17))
 (segment (start 89.9519 55.2162) (end 89.9519 45.98) (width 0.3) (layer "B.Cu") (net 17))
 (segment (start 88.62 56.5481) (end 89.9519 55.2162) (width 0.3) (layer "B.Cu") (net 17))
 (segment (start 88.62 58.25) (end 88.62 56.5481) (width 0.3) (layer "B.Cu") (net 17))
 (segment (start 91.75 80) (end 85 80) (width 0.3) (layer "F.Cu") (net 21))
 (segment locked (start 43.8 81.5) (end 36.18 81.5) (width 0.4) (layer "F.Cu") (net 11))
 (segment locked (start 39.29 76.5881) (end 36.18 79.6981) (width 0.4) (layer "B.Cu") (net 11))
 (segment locked (start 36.18 81.5) (end 36.18 79.6981) (width 0.4) (layer "B.Cu") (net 11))
 (segment locked (start 39.29 69.5) (end 39.29 76.5881) (width 0.4) (layer "B.Cu") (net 11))
 (segment (start 70 14) (end 75.38 14) (width 0.3) (layer "F.Cu") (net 12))
 (segment (start 68.13 38.9781) (end 71.25 42.0981) (width 0.3) (layer "B.Cu") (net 12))
 (segment (start 69.6895 20.8524) (end 68.13 22.4119) (width 0.3) (layer "B.Cu") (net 12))
 (segment (start 71.25 43.5) (end 71.25 42.0981) (width 0.3) (layer "B.Cu") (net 12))
 (segment (start 67.67 21.9519) (end 68.13 22.4119) (width 0.3) (layer "B.Cu") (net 12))
 (segment (start 76.1424 20.8524) (end 75.38 20.8524) (width 0.3) (layer "B.Cu") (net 12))
 (segment (start 75.38 20.8524) (end 69.6895 20.8524) (width 0.3) (layer "B.Cu") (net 12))
 (segment (start 68.13 22.4119) (end 68.13 31) (width 0.3) (layer "B.Cu") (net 12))
 (segment (start 68.13 31) (end 68.13 38.9781) (width 0.3) (layer "B.Cu") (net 12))
 (segment (start 80.79 25.5) (end 76.1424 20.8524) (width 0.3) (layer "B.Cu") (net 12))
 (segment (start 67.67 20.75) (end 67.67 21.9519) (width 0.3) (layer "B.Cu") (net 12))
 (segment (start 75.38 20.8524) (end 75.38 14) (width 0.3) (layer "B.Cu") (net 12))
 (segment (start 75.71 25.5) (end 74.6081 25.5) (width 0.3) (layer "F.Cu") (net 1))
 (segment (start 66.71 25.25) (end 67.9242 26.4642) (width 0.3) (layer "F.Cu") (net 1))
 (segment (start 73.6439 26.4642) (end 74.6081 25.5) (width 0.3) (layer "F.Cu") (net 1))
 (segment (start 64.2 64.655) (end 56.75 64.655) (width 0.3) (layer "F.Cu") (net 1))
 (segment (start 67.9242 26.4642) (end 73.6439 26.4642) (width 0.3) (layer "F.Cu") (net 1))
 (via (at 64.2 64.655) (size 0.8) (drill 0.4) (layers "F.Cu" "B.Cu") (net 1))
 (segment (start 64.2 27.76) (end 64.2 64.655) (width 0.3) (layer "B.Cu") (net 1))
 (segment (start 66.71 25.25) (end 64.2 27.76) (width 0.3) (layer "B.Cu") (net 1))
 (segment locked (start 37.865 64.655) (end 46.25 64.655) (width 0.4) (layer "F.Cu") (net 7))
 (segment locked (start 34.71 61.5) (end 37.865 64.655) (width 0.4) (layer "F.Cu") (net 7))
 (segment locked (start 34.71 61.5) (end 34.21 62) (width 0.4) (layer "B.Cu") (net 7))
 (segment locked (start 34.21 62) (end 34.21 69.5) (width 0.4) (layer "B.Cu") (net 7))
 (segment (start 105.29 34) (end 104.0881 34) (width 0.3) (layer "B.Cu") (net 25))
 (segment (start 94.58 24) (end 95.29 24) (width 0.3) (layer "B.Cu") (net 25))
 (segment (start 104.0881 32.7981) (end 104.0881 34) (width 0.3) (layer "B.Cu") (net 25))
 (segment (start 95.29 24) (end 104.0881 32.7981) (width 0.3) (layer "B.Cu") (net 25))
 (segment (start 95.67 39.25) (end 95.67 40.4519) (width 0.3) (layer "B.Cu") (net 23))
 (segment (start 97.75 42.5319) (end 97.75 46) (width 0.3) (layer "B.Cu") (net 23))
 (segment (start 95.67 40.4519) (end 97.75 42.5319) (width 0.3) (layer "B.Cu") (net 23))
 (segment (start 56.75 63.385) (end 59.4675 63.385) (width 0.3) (layer "F.Cu") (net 2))
 (segment (start 98.67 52.149) (end 98.67 52.75) (width 0.3) (layer "F.Cu") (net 2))
 (segment (start 59.4675 63.385) (end 70.1025 52.75) (width 0.3) (layer "F.Cu") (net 2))
 (segment (start 98.67 52.149) (end 98.67 51.5481) (width 0.3) (layer "F.Cu") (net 2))
 (segment (start 70.1025 52.75) (end 98.67 52.75) (width 0.3) (layer "F.Cu") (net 2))
 (segment (start 98.67 51.5481) (end 105.83 44.3881) (width 0.3) (layer "F.Cu") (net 2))
 (segment (start 105.83 44.3881) (end 105.83 39.25) (width 0.3) (layer "F.Cu") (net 2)))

